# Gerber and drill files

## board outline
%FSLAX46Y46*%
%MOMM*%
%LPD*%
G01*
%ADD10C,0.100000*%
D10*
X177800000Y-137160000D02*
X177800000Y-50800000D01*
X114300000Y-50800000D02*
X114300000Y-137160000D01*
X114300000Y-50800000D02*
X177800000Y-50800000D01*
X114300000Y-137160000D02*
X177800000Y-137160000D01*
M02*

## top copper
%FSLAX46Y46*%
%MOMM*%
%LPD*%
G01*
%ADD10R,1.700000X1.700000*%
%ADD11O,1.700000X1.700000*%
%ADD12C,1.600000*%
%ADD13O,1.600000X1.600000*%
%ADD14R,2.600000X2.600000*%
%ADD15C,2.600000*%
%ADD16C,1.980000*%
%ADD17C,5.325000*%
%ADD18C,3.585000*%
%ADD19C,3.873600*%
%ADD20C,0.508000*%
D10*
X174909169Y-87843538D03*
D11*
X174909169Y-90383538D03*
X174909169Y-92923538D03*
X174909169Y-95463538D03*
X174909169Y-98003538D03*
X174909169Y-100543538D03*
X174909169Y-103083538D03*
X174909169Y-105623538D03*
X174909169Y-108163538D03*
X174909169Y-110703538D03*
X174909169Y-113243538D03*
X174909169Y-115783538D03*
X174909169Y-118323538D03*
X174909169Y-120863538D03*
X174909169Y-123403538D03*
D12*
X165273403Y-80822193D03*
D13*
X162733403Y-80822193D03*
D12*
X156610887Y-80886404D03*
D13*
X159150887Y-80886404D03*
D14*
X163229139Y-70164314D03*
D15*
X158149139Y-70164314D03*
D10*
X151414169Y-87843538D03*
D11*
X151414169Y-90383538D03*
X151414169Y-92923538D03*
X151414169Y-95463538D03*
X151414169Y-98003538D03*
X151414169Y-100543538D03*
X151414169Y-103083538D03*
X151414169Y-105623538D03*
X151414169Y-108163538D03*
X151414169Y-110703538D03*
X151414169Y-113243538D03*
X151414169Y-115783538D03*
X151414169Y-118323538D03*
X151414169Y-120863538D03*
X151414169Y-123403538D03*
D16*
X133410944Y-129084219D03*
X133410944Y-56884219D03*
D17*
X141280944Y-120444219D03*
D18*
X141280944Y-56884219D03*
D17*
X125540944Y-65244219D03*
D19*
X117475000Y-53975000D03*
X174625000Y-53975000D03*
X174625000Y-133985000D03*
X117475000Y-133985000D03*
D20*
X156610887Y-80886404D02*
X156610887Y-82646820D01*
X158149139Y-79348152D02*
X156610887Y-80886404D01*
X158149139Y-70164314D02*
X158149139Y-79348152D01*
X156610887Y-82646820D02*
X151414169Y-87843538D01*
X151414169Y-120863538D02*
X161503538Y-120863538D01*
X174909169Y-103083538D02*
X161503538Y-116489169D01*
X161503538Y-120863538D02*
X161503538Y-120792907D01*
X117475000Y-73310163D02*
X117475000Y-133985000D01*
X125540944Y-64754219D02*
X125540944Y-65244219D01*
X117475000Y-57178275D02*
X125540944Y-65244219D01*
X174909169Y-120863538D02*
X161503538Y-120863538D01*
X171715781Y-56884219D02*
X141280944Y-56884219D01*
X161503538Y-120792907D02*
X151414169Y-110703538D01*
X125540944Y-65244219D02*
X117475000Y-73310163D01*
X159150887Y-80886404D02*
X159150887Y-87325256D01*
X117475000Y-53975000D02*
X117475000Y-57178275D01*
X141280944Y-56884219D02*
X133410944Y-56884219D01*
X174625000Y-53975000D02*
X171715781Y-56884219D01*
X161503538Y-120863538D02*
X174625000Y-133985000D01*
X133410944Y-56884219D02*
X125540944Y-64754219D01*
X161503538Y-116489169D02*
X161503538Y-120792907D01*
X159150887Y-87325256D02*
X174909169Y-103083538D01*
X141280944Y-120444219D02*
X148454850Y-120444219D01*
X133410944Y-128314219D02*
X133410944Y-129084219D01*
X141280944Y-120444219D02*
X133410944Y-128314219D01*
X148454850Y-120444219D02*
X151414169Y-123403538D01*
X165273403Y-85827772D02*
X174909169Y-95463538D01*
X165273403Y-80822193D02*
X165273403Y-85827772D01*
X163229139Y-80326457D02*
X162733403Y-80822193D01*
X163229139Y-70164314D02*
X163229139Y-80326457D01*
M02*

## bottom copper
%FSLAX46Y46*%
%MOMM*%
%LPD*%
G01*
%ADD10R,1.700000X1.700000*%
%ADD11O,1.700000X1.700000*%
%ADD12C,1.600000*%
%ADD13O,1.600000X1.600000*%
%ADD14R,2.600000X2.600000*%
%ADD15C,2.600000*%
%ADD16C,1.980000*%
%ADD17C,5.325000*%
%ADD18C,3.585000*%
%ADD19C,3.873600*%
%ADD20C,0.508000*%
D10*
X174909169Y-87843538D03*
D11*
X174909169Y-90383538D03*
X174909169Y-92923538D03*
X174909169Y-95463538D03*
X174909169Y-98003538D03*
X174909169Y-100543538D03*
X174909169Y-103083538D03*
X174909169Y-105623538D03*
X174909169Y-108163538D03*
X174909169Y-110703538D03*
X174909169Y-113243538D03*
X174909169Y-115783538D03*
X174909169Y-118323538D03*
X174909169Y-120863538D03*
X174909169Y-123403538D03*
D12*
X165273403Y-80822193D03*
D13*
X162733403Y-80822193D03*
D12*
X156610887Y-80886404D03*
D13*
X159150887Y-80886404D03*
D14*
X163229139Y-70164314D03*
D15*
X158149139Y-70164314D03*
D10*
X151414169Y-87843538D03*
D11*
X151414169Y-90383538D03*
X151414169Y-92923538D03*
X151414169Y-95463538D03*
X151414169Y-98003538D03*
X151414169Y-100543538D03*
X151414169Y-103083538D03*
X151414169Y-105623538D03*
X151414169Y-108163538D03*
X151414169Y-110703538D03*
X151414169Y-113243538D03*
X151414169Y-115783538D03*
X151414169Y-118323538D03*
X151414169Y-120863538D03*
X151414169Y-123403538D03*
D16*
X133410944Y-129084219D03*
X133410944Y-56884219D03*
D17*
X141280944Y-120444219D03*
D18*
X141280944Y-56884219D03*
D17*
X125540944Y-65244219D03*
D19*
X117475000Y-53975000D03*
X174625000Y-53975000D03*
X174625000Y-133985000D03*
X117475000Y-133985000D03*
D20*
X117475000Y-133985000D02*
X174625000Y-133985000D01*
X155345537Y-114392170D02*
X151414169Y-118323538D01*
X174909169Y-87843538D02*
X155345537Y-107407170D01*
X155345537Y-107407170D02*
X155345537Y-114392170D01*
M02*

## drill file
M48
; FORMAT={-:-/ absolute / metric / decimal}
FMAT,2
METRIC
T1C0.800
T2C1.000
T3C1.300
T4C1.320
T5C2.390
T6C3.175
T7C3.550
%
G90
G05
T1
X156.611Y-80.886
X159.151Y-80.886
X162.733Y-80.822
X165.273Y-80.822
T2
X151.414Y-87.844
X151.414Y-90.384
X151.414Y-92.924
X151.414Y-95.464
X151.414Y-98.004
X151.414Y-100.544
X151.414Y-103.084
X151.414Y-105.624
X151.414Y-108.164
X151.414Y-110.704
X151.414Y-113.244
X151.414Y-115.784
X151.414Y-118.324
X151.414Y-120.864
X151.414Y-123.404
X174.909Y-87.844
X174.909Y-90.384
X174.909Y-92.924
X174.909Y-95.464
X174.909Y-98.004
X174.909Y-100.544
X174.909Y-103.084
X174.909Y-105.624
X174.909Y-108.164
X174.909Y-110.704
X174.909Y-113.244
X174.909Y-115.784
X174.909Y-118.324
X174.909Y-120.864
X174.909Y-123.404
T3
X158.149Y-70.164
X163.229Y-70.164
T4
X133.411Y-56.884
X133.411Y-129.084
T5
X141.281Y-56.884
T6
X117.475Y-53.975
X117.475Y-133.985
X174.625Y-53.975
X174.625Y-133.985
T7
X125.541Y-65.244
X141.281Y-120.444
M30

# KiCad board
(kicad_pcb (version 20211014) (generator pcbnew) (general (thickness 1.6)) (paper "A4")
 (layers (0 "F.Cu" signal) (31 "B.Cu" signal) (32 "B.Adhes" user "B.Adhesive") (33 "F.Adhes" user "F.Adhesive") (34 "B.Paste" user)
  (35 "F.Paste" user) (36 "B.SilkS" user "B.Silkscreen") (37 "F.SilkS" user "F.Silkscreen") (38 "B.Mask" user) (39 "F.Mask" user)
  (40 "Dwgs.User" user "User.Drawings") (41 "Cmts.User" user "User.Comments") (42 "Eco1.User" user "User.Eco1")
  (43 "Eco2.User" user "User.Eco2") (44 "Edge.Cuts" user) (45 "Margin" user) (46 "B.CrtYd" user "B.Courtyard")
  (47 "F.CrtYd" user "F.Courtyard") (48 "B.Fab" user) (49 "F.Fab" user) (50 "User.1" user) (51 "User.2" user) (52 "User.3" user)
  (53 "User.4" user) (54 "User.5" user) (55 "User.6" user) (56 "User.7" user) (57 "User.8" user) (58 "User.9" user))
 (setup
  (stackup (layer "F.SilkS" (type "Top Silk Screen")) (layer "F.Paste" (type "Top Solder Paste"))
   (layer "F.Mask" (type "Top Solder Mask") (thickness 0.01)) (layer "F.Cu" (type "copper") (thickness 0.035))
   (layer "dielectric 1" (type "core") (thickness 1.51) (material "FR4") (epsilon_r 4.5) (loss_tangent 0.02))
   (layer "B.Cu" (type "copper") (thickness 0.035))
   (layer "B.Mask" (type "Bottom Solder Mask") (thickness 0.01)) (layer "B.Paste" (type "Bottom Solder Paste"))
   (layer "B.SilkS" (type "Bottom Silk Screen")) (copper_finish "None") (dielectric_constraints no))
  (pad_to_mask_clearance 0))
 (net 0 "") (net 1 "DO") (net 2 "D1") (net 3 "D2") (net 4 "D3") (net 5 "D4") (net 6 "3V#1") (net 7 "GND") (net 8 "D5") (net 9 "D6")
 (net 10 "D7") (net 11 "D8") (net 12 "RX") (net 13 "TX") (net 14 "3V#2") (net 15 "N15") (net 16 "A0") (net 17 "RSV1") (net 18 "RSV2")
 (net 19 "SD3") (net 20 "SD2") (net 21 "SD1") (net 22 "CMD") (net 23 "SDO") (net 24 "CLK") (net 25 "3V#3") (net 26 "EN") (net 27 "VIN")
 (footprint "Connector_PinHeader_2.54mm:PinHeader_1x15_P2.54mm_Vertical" (layer "F.Cu") (at 174.909169 87.843538)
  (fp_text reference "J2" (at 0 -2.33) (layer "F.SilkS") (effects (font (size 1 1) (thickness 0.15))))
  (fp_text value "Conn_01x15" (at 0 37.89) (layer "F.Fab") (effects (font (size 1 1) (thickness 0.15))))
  (pad "1" thru_hole rect locked (at 0 0) (size 1.7 1.7) (drill 1) (layers *.Cu *.Mask) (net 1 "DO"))
  (pad "2" thru_hole oval locked (at 0 2.54) (size 1.7 1.7) (drill 1) (layers *.Cu *.Mask) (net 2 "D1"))
  (pad "3" thru_hole oval locked (at 0 5.08) (size 1.7 1.7) (drill 1) (layers *.Cu *.Mask) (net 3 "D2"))
  (pad "4" thru_hole oval locked (at 0 7.62) (size 1.7 1.7) (drill 1) (layers *.Cu *.Mask) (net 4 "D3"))
  (pad "5" thru_hole oval locked (at 0 10.16) (size 1.7 1.7) (drill 1) (layers *.Cu *.Mask) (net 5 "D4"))
  (pad "6" thru_hole oval locked (at 0 12.7) (size 1.7 1.7) (drill 1) (layers *.Cu *.Mask) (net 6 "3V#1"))
  (pad "7" thru_hole oval locked (at 0 15.24) (size 1.7 1.7) (drill 1) (layers *.Cu *.Mask) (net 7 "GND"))
  (pad "8" thru_hole oval locked (at 0 17.78) (size 1.7 1.7) (drill 1) (layers *.Cu *.Mask) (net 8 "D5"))
  (pad "9" thru_hole oval locked (at 0 20.32) (size 1.7 1.7) (drill 1) (layers *.Cu *.Mask) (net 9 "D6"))
  (pad "10" thru_hole oval locked (at 0 22.86) (size 1.7 1.7) (drill 1) (layers *.Cu *.Mask) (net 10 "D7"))
  (pad "11" thru_hole oval locked (at 0 25.4) (size 1.7 1.7) (drill 1) (layers *.Cu *.Mask) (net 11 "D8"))
  (pad "12" thru_hole oval locked (at 0 27.94) (size 1.7 1.7) (drill 1) (layers *.Cu *.Mask) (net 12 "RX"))
  (pad "13" thru_hole oval locked (at 0 30.48) (size 1.7 1.7) (drill 1) (layers *.Cu *.Mask) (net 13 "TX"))
  (pad "14" thru_hole oval locked (at 0 33.02) (size 1.7 1.7) (drill 1) (layers *.Cu *.Mask) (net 7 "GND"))
  (pad "15" thru_hole oval locked (at 0 35.56) (size 1.7 1.7) (drill 1) (layers *.Cu *.Mask) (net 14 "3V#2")))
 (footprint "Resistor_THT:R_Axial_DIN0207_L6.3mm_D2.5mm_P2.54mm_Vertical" (layer "F.Cu") (at 165.273403 80.822193 180)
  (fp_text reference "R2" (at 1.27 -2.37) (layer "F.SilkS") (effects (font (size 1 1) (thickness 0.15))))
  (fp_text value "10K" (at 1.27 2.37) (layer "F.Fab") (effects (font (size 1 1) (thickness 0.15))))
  (pad "1" thru_hole circle locked (at 0 0 180) (size 1.6 1.6) (drill 0.8) (layers *.Cu *.Mask) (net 4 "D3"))
  (pad "2" thru_hole oval locked (at 2.54 0 180) (size 1.6 1.6) (drill 0.8) (layers *.Cu *.Mask) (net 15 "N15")))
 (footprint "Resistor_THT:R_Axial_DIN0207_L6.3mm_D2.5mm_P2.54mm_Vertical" (layer "F.Cu") (at 156.610887 80.886404)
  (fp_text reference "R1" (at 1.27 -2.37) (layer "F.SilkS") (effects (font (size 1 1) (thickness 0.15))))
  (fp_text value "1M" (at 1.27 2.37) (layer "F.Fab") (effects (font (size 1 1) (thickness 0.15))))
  (pad "1" thru_hole circle locked (at 0 0) (size 1.6 1.6) (drill 0.8) (layers *.Cu *.Mask) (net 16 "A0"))
  (pad "2" thru_hole oval locked (at 2.54 0) (size 1.6 1.6) (drill 0.8) (layers *.Cu *.Mask) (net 7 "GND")))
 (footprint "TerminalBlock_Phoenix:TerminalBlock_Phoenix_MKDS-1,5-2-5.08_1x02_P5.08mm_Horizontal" (layer "F.Cu")
  (at 163.229139 70.164314 180)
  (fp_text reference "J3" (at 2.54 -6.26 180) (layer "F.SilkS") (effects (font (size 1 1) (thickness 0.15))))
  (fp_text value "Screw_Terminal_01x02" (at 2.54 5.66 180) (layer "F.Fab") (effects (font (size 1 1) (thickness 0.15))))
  (pad "1" thru_hole rect locked (at 0 0 180) (size 2.6 2.6) (drill 1.3) (layers *.Cu *.Mask) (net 15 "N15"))
  (pad "2" thru_hole circle locked (at 5.08 0 180) (size 2.6 2.6) (drill 1.3) (layers *.Cu *.Mask) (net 16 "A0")))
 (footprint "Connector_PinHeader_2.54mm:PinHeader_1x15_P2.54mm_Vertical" (layer "F.Cu") (at 151.414169 87.843538)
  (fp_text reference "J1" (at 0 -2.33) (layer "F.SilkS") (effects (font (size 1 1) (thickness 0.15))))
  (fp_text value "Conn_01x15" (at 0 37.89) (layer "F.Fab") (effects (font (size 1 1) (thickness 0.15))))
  (pad "1" thru_hole rect locked (at 0 0) (size 1.7 1.7) (drill 1) (layers *.Cu *.Mask) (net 16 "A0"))
  (pad "2" thru_hole oval locked (at 0 2.54) (size 1.7 1.7) (drill 1) (layers *.Cu *.Mask) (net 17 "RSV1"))
  (pad "3" thru_hole oval locked (at 0 5.08) (size 1.7 1.7) (drill 1) (layers *.Cu *.Mask) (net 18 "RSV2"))
  (pad "4" thru_hole oval locked (at 0 7.62) (size 1.7 1.7) (drill 1) (layers *.Cu *.Mask) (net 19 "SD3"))
  (pad "5" thru_hole oval locked (at 0 10.16) (size 1.7 1.7) (drill 1) (layers *.Cu *.Mask) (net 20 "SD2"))
  (pad "6" thru_hole oval locked (at 0 12.7) (size 1.7 1.7) (drill 1) (layers *.Cu *.Mask) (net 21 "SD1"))
  (pad "7" thru_hole oval locked (at 0 15.24) (size 1.7 1.7) (drill 1) (layers *.Cu *.Mask) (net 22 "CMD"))
  (pad "8" thru_hole oval locked (at 0 17.78) (size 1.7 1.7) (drill 1) (layers *.Cu *.Mask) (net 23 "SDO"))
  (pad "9" thru_hole oval locked (at 0 20.32) (size 1.7 1.7) (drill 1) (layers *.Cu *.Mask) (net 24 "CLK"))
  (pad "10" thru_hole oval locked (at 0 22.86) (size 1.7 1.7) (drill 1) (layers *.Cu *.Mask) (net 7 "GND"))
  (pad "11" thru_hole oval locked (at 0 25.4) (size 1.7 1.7) (drill 1) (layers *.Cu *.Mask) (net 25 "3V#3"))
  (pad "12" thru_hole oval locked (at 0 27.94) (size 1.7 1.7) (drill 1) (layers *.Cu *.Mask) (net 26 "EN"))
  (pad "13" thru_hole oval locked (at 0 30.48) (size 1.7 1.7) (drill 1) (layers *.Cu *.Mask) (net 1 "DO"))
  (pad "14" thru_hole oval locked (at 0 33.02) (size 1.7 1.7) (drill 1) (layers *.Cu *.Mask) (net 7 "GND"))
  (pad "15" thru_hole oval locked (at 0 35.56) (size 1.7 1.7) (drill 1) (layers *.Cu *.Mask) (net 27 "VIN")))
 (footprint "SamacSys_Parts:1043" (layer "F.Cu") (at 133.410944 129.084219 90)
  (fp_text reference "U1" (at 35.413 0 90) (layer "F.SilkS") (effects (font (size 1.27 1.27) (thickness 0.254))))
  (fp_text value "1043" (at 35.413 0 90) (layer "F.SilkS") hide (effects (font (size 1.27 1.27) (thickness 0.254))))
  (pad "1" thru_hole circle locked (at 0 0 90) (size 1.98 1.98) (drill 1.32) (layers *.Cu *.Mask) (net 27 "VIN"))
  (pad "2" thru_hole circle locked (at 72.2 0 90) (size 1.98 1.98) (drill 1.32) (layers *.Cu *.Mask) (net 7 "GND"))
  (pad "MH1" thru_hole circle locked (at 8.64 7.87 90) (size 5.325 5.325) (drill 3.55) (layers *.Cu *.Mask) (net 27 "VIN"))
  (pad "MH2" thru_hole circle locked (at 72.2 7.87 90) (size 3.585 3.585) (drill 2.39) (layers *.Cu *.Mask) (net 7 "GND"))
  (pad "MH3" thru_hole circle locked (at 63.84 -7.87 90) (size 5.325 5.325) (drill 3.55) (layers *.Cu *.Mask) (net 7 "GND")))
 (gr_line (start 177.8 137.16) (end 177.8 50.8) (layer "Edge.Cuts") (width 0.1))
 (gr_line (start 114.3 50.8) (end 114.3 137.16) (layer "Edge.Cuts") (width 0.1))
 (gr_line (start 114.3 50.8) (end 177.8 50.8) (layer "Edge.Cuts") (width 0.1))
 (gr_line (start 114.3 137.16) (end 177.8 137.16) (layer "Edge.Cuts") (width 0.1))
 (segment (start 156.610887 80.886404) (end 156.610887 82.64682) (width 0.508) (layer "F.Cu") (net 16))
 (segment (start 158.149139 79.348152) (end 156.610887 80.886404) (width 0.508) (layer "F.Cu") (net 16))
 (segment (start 158.149139 70.164314) (end 158.149139 79.348152) (width 0.508) (layer "F.Cu") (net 16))
 (segment (start 156.610887 82.64682) (end 151.414169 87.843538) (width 0.508) (layer "F.Cu") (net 16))
 (segment (start 151.414169 120.863538) (end 161.503538 120.863538) (width 0.508) (layer "F.Cu") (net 7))
 (segment (start 174.909169 103.083538) (end 161.503538 116.489169) (width 0.508) (layer "F.Cu") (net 7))
 (segment (start 161.503538 120.863538) (end 161.503538 120.792907) (width 0.508) (layer "F.Cu") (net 7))
 (segment (start 117.475 73.310163) (end 117.475 133.985) (width 0.508) (layer "F.Cu") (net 7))
 (segment (start 125.540944 64.754219) (end 125.540944 65.244219) (width 0.508) (layer "F.Cu") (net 7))
 (segment (start 117.475 57.178275) (end 125.540944 65.244219) (width 0.508) (layer "F.Cu") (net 7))
 (segment (start 174.909169 120.863538) (end 161.503538 120.863538) (width 0.508) (layer "F.Cu") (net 7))
 (segment (start 171.715781 56.884219) (end 141.280944 56.884219) (width 0.508) (layer "F.Cu") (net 7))
 (segment (start 161.503538 120.792907) (end 151.414169 110.703538) (width 0.508) (layer "F.Cu") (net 7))
 (segment (start 125.540944 65.244219) (end 117.475 73.310163) (width 0.508) (layer "F.Cu") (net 7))
 (segment (start 159.150887 80.886404) (end 159.150887 87.325256) (width 0.508) (layer "F.Cu") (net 7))
 (segment (start 117.475 53.975) (end 117.475 57.178275) (width 0.508) (layer "F.Cu") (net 7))
 (segment (start 141.280944 56.884219) (end 133.410944 56.884219) (width 0.508) (layer "F.Cu") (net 7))
 (segment (start 174.625 53.975) (end 171.715781 56.884219) (width 0.508) (layer "F.Cu") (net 7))
 (segment (start 161.503538 120.863538) (end 174.625 133.985) (width 0.508) (layer "F.Cu") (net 7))
 (segment (start 133.410944 56.884219) (end 125.540944 64.754219) (width 0.508) (layer "F.Cu") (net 7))
 (segment (start 161.503538 116.489169) (end 161.503538 120.792907) (width 0.508) (layer "F.Cu") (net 7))
 (segment (start 159.150887 87.325256) (end 174.909169 103.083538) (width 0.508) (layer "F.Cu") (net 7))
 (via (at 117.475 53.975) (size 3.8736) (drill 3.175) (layers "F.Cu" "B.Cu") (free) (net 7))
 (via (at 174.625 53.975) (size 3.8736) (drill 3.175) (layers "F.Cu" "B.Cu") (free) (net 7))
 (via (at 174.625 133.985) (size 3.8736) (drill 3.175) (layers "F.Cu" "B.Cu") (free) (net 7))
 (via (at 117.475 133.985) (size 3.8736) (drill 3.175) (layers "F.Cu" "B.Cu") (free) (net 7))
 (segment (start 117.475 133.985) (end 174.625 133.985) (width 0.508) (layer "B.Cu") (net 7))
 (segment (start 155.345537 114.39217) (end 151.414169 118.323538) (width 0.508) (layer "B.Cu") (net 1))
 (segment (start 174.909169 87.843538) (end 155.345537 107.40717) (width 0.508) (layer "B.Cu") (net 1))
 (segment (start 155.345537 107.40717) (end 155.345537 114.39217) (width 0.508) (layer "B.Cu") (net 1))
 (segment (start 141.280944 120.444219) (end 148.45485 120.444219) (width 0.508) (layer "F.Cu") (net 27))
 (segment (start 133.410944 128.314219) (end 133.410944 129.084219) (width 0.508) (layer "F.Cu") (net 27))
 (segment (start 141.280944 120.444219) (end 133.410944 128.314219) (width 0.508) (layer "F.Cu") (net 27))
 (segment (start 148.45485 120.444219) (end 151.414169 123.403538) (width 0.508) (layer "F.Cu") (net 27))
 (segment (start 165.273403 85.827772) (end 174.909169 95.463538) (width 0.508) (layer "F.Cu") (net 4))
 (segment (start 165.273403 80.822193) (end 165.273403 85.827772) (width 0.508) (layer "F.Cu") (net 4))
 (segment (start 163.229139 80.326457) (end 162.733403 80.822193) (width 0.508) (layer "F.Cu") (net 15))
 (segment (start 163.229139 70.164314) (end 163.229139 80.326457) (width 0.508) (layer "F.Cu") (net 15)))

